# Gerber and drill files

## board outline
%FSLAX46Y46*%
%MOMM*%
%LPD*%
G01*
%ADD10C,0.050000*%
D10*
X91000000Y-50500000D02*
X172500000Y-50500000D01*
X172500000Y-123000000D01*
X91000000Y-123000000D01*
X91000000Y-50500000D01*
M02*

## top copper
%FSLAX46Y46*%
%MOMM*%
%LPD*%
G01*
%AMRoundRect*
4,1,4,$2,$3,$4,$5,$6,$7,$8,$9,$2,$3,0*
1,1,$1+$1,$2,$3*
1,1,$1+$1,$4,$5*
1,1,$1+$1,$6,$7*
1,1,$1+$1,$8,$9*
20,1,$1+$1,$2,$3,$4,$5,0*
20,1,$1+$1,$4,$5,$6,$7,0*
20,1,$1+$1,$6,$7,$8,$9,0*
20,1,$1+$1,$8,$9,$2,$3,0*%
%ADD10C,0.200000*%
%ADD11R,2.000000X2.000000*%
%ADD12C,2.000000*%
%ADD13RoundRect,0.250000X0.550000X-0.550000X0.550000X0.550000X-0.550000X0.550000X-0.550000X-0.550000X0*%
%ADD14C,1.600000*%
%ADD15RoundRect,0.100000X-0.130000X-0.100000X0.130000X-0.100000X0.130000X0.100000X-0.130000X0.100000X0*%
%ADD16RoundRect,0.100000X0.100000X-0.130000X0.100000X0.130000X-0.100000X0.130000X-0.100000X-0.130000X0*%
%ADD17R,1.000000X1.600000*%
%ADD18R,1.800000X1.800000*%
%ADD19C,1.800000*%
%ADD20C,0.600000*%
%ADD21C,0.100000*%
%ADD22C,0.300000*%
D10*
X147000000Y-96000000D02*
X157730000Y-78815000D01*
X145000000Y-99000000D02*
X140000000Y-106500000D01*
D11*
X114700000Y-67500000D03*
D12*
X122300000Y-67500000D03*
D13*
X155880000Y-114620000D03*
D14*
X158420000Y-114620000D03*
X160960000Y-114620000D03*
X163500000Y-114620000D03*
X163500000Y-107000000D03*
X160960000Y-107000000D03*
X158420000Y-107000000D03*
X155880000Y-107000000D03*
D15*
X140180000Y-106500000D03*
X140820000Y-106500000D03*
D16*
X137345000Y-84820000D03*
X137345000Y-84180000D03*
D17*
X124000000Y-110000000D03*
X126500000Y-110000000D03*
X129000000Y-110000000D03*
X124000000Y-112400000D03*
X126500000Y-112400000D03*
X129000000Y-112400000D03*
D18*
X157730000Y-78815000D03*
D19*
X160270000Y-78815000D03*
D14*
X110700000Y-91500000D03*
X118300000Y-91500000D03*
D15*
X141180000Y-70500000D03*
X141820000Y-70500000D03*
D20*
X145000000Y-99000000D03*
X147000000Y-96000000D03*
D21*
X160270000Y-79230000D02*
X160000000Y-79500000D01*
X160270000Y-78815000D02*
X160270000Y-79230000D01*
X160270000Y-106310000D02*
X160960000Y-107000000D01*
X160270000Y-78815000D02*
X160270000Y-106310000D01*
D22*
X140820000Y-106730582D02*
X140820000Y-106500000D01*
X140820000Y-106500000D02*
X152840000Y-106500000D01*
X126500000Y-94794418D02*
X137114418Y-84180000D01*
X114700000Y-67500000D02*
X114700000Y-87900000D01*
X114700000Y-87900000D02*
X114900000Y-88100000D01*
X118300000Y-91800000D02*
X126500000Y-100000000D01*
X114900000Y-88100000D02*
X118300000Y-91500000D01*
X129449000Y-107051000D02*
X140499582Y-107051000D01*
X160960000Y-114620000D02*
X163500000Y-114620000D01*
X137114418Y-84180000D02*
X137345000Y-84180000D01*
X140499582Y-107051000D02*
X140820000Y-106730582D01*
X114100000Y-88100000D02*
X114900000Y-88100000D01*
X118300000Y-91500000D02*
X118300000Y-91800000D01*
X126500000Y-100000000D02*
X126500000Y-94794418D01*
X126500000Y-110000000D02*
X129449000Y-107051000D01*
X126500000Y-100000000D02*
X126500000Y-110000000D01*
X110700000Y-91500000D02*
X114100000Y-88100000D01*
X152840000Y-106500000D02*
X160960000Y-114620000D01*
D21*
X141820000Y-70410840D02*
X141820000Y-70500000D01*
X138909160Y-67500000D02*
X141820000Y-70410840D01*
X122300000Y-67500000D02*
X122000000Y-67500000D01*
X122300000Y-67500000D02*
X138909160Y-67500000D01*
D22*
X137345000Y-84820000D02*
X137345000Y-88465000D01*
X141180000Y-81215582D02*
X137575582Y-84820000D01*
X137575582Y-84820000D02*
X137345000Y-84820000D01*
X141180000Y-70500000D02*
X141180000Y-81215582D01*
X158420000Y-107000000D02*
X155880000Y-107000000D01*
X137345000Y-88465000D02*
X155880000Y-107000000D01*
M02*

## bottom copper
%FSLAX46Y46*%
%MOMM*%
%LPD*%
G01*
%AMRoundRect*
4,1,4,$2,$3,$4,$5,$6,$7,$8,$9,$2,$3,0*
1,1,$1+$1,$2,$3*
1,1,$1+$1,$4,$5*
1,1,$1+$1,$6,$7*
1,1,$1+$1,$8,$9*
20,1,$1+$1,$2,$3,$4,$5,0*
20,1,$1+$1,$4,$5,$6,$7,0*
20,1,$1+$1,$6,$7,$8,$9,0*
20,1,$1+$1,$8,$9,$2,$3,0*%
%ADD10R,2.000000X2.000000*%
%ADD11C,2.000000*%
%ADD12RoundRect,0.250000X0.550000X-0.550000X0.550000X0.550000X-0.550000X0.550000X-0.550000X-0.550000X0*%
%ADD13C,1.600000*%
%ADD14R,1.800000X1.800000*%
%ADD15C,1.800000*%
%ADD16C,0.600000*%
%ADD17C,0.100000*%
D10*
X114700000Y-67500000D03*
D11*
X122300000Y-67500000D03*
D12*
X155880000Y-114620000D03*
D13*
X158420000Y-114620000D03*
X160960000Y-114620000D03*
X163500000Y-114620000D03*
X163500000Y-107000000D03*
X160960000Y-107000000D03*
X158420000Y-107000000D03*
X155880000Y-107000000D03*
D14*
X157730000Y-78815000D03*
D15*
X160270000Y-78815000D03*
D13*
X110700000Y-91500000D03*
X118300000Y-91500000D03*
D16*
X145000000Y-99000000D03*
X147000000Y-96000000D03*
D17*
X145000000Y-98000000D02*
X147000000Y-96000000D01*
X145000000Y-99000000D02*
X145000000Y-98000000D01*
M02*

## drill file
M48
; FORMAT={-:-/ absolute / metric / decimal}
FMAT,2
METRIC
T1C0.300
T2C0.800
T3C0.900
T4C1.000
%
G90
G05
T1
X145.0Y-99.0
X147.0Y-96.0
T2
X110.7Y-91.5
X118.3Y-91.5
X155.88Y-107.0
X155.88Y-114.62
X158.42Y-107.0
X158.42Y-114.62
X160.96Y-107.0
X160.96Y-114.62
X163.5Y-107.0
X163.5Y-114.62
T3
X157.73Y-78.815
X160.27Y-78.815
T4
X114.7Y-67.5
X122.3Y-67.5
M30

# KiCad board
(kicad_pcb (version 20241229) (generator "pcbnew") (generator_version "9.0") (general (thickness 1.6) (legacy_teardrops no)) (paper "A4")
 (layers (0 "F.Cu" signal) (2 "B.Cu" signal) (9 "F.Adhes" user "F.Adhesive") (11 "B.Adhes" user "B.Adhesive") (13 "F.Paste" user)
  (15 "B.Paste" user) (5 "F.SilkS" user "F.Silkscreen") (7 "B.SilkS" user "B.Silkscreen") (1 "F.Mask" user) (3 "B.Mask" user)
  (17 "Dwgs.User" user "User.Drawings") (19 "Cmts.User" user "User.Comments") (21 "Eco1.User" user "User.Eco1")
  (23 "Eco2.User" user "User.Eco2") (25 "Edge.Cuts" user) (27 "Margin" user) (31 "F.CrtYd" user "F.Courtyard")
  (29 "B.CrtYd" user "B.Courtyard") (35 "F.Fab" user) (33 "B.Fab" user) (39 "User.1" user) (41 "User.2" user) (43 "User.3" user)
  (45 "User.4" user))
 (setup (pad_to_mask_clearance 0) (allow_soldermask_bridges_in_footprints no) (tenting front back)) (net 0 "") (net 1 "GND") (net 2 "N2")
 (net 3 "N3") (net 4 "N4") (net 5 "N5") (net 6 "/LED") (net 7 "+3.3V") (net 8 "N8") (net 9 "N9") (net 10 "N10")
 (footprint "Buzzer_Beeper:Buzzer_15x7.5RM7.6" (layer "F.Cu") (at 114.7 67.5)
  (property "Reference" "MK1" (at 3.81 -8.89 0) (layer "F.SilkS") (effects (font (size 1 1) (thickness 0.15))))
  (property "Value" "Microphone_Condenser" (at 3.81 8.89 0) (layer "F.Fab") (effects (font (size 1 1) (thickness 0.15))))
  (pad "1" thru_hole rect (at 0 0) (size 2 2) (drill 1) (layers "*.Cu" "*.Mask") (remove_unused_layers no) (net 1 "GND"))
  (pad "2" thru_hole circle (at 7.6 0) (size 2 2) (drill 1) (layers "*.Cu" "*.Mask") (remove_unused_layers no) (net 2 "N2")))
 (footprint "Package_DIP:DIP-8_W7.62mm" (layer "F.Cu") (at 155.88 114.62 90)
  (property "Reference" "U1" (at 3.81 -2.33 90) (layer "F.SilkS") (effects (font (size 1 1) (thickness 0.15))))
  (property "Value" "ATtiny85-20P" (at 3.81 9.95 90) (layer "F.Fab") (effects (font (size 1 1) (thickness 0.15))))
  (pad "1" thru_hole roundrect (at 0 0 90) (size 1.6 1.6) (drill 0.8) (layers "*.Cu" "*.Mask") (remove_unused_layers no)
   (roundrect_rratio 0.15625) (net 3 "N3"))
  (pad "2" thru_hole circle (at 0 2.54 90) (size 1.6 1.6) (drill 0.8) (layers "*.Cu" "*.Mask") (remove_unused_layers no) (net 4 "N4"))
  (pad "3" thru_hole circle (at 0 5.08 90) (size 1.6 1.6) (drill 0.8) (layers "*.Cu" "*.Mask") (remove_unused_layers no) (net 1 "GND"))
  (pad "4" thru_hole circle (at 0 7.62 90) (size 1.6 1.6) (drill 0.8) (layers "*.Cu" "*.Mask") (remove_unused_layers no) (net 1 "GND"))
  (pad "5" thru_hole circle (at 7.62 7.62 90) (size 1.6 1.6) (drill 0.8) (layers "*.Cu" "*.Mask") (remove_unused_layers no) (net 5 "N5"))
  (pad "6" thru_hole circle (at 7.62 5.08 90) (size 1.6 1.6) (drill 0.8) (layers "*.Cu" "*.Mask") (remove_unused_layers no) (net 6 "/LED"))
  (pad "7" thru_hole circle (at 7.62 2.54 90) (size 1.6 1.6) (drill 0.8) (layers "*.Cu" "*.Mask") (remove_unused_layers no) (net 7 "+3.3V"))
  (pad "8" thru_hole circle (at 7.62 0 90) (size 1.6 1.6) (drill 0.8) (layers "*.Cu" "*.Mask") (remove_unused_layers no) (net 7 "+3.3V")))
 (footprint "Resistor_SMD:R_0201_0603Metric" (layer "F.Cu") (at 140.5 106.5)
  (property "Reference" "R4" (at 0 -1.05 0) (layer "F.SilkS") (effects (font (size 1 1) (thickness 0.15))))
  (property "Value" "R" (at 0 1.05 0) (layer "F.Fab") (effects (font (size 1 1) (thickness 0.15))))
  (pad "" smd roundrect (at -0.345 0) (size 0.318 0.36) (layers "F.Paste") (roundrect_rratio 0.25))
  (pad "" smd roundrect (at 0.345 0) (size 0.318 0.36) (layers "F.Paste") (roundrect_rratio 0.25))
  (pad "1" smd roundrect (at -0.32 0) (size 0.46 0.4) (layers "F.Cu" "F.Mask") (roundrect_rratio 0.25) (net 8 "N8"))
  (pad "2" smd roundrect (at 0.32 0) (size 0.46 0.4) (layers "F.Cu" "F.Mask") (roundrect_rratio 0.25) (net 1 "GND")))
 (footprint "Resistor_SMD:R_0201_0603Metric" (layer "F.Cu") (at 137.345 84.5 90)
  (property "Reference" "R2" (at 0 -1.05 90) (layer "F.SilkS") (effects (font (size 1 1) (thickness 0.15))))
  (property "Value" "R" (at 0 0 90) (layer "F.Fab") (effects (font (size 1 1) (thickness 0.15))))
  (pad "" smd roundrect (at -0.345 0 90) (size 0.318 0.36) (layers "F.Paste") (roundrect_rratio 0.25))
  (pad "" smd roundrect (at 0.345 0 90) (size 0.318 0.36) (layers "F.Paste") (roundrect_rratio 0.25))
  (pad "1" smd roundrect (at -0.32 0 90) (size 0.46 0.4) (layers "F.Cu" "F.Mask") (roundrect_rratio 0.25) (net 7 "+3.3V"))
  (pad "2" smd roundrect (at 0.32 0 90) (size 0.46 0.4) (layers "F.Cu" "F.Mask") (roundrect_rratio 0.25) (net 1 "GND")))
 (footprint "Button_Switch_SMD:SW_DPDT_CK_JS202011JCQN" (layer "F.Cu") (at 126.5 111.2)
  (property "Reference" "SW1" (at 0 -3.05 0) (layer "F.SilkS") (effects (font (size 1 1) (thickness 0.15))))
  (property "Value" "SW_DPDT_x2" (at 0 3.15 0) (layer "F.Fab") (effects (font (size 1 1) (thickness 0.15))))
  (pad "1" smd rect (at -2.5 -1.2) (size 1 1.6) (layers "F.Cu" "F.Mask" "F.Paste") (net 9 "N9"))
  (pad "2" smd rect (at 0 -1.2) (size 1 1.6) (layers "F.Cu" "F.Mask" "F.Paste") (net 1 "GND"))
  (pad "3" smd rect (at 2.5 -1.2) (size 1 1.6) (layers "F.Cu" "F.Mask" "F.Paste") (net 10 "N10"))
  (pad "4" smd rect (at -2.5 1.2) (size 1 1.6) (layers "F.Cu" "F.Mask" "F.Paste"))
  (pad "5" smd rect (at 0 1.2) (size 1 1.6) (layers "F.Cu" "F.Mask" "F.Paste"))
  (pad "6" smd rect (at 2.5 1.2) (size 1 1.6) (layers "F.Cu" "F.Mask" "F.Paste")))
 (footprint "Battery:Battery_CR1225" (layer "F.Cu") (at 154 64)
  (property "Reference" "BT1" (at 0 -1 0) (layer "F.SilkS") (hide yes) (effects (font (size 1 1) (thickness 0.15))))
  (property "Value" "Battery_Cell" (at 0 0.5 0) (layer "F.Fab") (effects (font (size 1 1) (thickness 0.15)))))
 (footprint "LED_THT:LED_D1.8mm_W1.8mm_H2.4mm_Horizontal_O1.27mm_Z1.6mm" (layer "F.Cu") (at 157.73 78.815)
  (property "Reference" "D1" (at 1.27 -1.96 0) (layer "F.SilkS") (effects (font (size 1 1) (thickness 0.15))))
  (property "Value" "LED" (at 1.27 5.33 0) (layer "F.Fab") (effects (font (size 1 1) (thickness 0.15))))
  (pad "1" thru_hole rect (at 0 0) (size 1.8 1.8) (drill 0.9) (layers "*.Cu" "*.Mask") (remove_unused_layers no) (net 8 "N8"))
  (pad "2" thru_hole circle (at 2.54 0) (size 1.8 1.8) (drill 0.9) (layers "*.Cu" "*.Mask") (remove_unused_layers no) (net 6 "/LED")))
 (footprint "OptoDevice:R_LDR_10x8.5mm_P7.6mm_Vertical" (layer "F.Cu") (at 110.7 91.5)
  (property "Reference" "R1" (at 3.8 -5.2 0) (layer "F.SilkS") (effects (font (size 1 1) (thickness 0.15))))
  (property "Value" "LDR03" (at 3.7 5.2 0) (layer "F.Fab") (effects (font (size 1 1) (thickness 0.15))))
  (pad "1" thru_hole circle (at 0 0) (size 1.6 1.6) (drill 0.8) (layers "*.Cu" "*.Mask") (remove_unused_layers no) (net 1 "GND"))
  (pad "2" thru_hole circle (at 7.6 0) (size 1.6 1.6) (drill 0.8) (layers "*.Cu" "*.Mask") (remove_unused_layers no) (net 1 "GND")))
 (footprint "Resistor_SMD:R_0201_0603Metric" (layer "F.Cu") (at 141.5 70.5)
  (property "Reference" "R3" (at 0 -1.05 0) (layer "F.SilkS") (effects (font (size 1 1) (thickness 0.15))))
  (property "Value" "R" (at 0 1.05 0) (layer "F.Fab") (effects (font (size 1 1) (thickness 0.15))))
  (pad "" smd roundrect (at -0.345 0) (size 0.318 0.36) (layers "F.Paste") (roundrect_rratio 0.25))
  (pad "" smd roundrect (at 0.345 0) (size 0.318 0.36) (layers "F.Paste") (roundrect_rratio 0.25))
  (pad "1" smd roundrect (at -0.32 0) (size 0.46 0.4) (layers "F.Cu" "F.Mask") (roundrect_rratio 0.25) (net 7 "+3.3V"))
  (pad "2" smd roundrect (at 0.32 0) (size 0.46 0.4) (layers "F.Cu" "F.Mask") (roundrect_rratio 0.25) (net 2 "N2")))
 (gr_line (start 147 96) (end 157.73 78.815) (stroke (width 0.2) (type default)) (layer "F.Cu") (net 8))
 (gr_line (start 145 99) (end 140 106.5) (stroke (width 0.2) (type default)) (layer "F.Cu") (net 8))
 (gr_rect (start 91 50.5) (end 172.5 123) (stroke (width 0.05) (type default)) (fill no) (layer "Edge.Cuts"))
 (via (at 145 99) (size 0.6) (drill 0.3) (layers "F.Cu" "B.Cu") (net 8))
 (via (at 147 96) (size 0.6) (drill 0.3) (layers "F.Cu" "B.Cu") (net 8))
 (segment (start 145 98) (end 147 96) (width 0.1) (layer "B.Cu") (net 8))
 (segment (start 145 99) (end 145 98) (width 0.1) (layer "B.Cu") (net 8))
 (segment (start 160.27 79.23) (end 160 79.5) (width 0.1) (layer "F.Cu") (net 6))
 (segment (start 160.27 78.815) (end 160.27 79.23) (width 0.1) (layer "F.Cu") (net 6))
 (segment (start 160.27 106.31) (end 160.96 107) (width 0.1) (layer "F.Cu") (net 6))
 (segment (start 160.27 78.815) (end 160.27 106.31) (width 0.1) (layer "F.Cu") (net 6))
 (segment (start 140.82 106.730582) (end 140.82 106.5) (width 0.3) (layer "F.Cu") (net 1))
 (segment (start 140.82 106.5) (end 152.84 106.5) (width 0.3) (layer "F.Cu") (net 1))
 (segment (start 126.5 94.794418) (end 137.114418 84.18) (width 0.3) (layer "F.Cu") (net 1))
 (segment (start 114.7 67.5) (end 114.7 87.9) (width 0.3) (layer "F.Cu") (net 1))
 (segment (start 114.7 87.9) (end 114.9 88.1) (width 0.3) (layer "F.Cu") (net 1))
 (segment (start 118.3 91.8) (end 126.5 100) (width 0.3) (layer "F.Cu") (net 1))
 (segment (start 114.9 88.1) (end 118.3 91.5) (width 0.3) (layer "F.Cu") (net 1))
 (segment (start 129.449 107.051) (end 140.499582 107.051) (width 0.3) (layer "F.Cu") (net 1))
 (segment (start 160.96 114.62) (end 163.5 114.62) (width 0.3) (layer "F.Cu") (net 1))
 (segment (start 137.114418 84.18) (end 137.345 84.18) (width 0.3) (layer "F.Cu") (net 1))
 (segment (start 140.499582 107.051) (end 140.82 106.730582) (width 0.3) (layer "F.Cu") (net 1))
 (segment (start 114.1 88.1) (end 114.9 88.1) (width 0.3) (layer "F.Cu") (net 1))
 (segment (start 118.3 91.5) (end 118.3 91.8) (width 0.3) (layer "F.Cu") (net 1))
 (segment (start 126.5 100) (end 126.5 94.794418) (width 0.3) (layer "F.Cu") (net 1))
 (segment (start 126.5 110) (end 129.449 107.051) (width 0.3) (layer "F.Cu") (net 1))
 (segment (start 126.5 100) (end 126.5 110) (width 0.3) (layer "F.Cu") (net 1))
 (segment (start 110.7 91.5) (end 114.1 88.1) (width 0.3) (layer "F.Cu") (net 1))
 (segment (start 152.84 106.5) (end 160.96 114.62) (width 0.3) (layer "F.Cu") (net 1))
 (segment (start 141.82 70.41084) (end 141.82 70.5) (width 0.1) (layer "F.Cu") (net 2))
 (segment (start 138.90916 67.5) (end 141.82 70.41084) (width 0.1) (layer "F.Cu") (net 2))
 (segment (start 122.3 67.5) (end 122 67.5) (width 0.1) (layer "F.Cu") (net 2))
 (segment (start 122.3 67.5) (end 138.90916 67.5) (width 0.1) (layer "F.Cu") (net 2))
 (segment (start 137.345 84.82) (end 137.345 88.465) (width 0.3) (layer "F.Cu") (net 7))
 (segment (start 141.18 81.215582) (end 137.575582 84.82) (width 0.3) (layer "F.Cu") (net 7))
 (segment (start 137.575582 84.82) (end 137.345 84.82) (width 0.3) (layer "F.Cu") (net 7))
 (segment (start 141.18 70.5) (end 141.18 81.215582) (width 0.3) (layer "F.Cu") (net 7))
 (segment (start 158.42 107) (end 155.88 107) (width 0.3) (layer "F.Cu") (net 7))
 (segment (start 137.345 88.465) (end 155.88 107) (width 0.3) (layer "F.Cu") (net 7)))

